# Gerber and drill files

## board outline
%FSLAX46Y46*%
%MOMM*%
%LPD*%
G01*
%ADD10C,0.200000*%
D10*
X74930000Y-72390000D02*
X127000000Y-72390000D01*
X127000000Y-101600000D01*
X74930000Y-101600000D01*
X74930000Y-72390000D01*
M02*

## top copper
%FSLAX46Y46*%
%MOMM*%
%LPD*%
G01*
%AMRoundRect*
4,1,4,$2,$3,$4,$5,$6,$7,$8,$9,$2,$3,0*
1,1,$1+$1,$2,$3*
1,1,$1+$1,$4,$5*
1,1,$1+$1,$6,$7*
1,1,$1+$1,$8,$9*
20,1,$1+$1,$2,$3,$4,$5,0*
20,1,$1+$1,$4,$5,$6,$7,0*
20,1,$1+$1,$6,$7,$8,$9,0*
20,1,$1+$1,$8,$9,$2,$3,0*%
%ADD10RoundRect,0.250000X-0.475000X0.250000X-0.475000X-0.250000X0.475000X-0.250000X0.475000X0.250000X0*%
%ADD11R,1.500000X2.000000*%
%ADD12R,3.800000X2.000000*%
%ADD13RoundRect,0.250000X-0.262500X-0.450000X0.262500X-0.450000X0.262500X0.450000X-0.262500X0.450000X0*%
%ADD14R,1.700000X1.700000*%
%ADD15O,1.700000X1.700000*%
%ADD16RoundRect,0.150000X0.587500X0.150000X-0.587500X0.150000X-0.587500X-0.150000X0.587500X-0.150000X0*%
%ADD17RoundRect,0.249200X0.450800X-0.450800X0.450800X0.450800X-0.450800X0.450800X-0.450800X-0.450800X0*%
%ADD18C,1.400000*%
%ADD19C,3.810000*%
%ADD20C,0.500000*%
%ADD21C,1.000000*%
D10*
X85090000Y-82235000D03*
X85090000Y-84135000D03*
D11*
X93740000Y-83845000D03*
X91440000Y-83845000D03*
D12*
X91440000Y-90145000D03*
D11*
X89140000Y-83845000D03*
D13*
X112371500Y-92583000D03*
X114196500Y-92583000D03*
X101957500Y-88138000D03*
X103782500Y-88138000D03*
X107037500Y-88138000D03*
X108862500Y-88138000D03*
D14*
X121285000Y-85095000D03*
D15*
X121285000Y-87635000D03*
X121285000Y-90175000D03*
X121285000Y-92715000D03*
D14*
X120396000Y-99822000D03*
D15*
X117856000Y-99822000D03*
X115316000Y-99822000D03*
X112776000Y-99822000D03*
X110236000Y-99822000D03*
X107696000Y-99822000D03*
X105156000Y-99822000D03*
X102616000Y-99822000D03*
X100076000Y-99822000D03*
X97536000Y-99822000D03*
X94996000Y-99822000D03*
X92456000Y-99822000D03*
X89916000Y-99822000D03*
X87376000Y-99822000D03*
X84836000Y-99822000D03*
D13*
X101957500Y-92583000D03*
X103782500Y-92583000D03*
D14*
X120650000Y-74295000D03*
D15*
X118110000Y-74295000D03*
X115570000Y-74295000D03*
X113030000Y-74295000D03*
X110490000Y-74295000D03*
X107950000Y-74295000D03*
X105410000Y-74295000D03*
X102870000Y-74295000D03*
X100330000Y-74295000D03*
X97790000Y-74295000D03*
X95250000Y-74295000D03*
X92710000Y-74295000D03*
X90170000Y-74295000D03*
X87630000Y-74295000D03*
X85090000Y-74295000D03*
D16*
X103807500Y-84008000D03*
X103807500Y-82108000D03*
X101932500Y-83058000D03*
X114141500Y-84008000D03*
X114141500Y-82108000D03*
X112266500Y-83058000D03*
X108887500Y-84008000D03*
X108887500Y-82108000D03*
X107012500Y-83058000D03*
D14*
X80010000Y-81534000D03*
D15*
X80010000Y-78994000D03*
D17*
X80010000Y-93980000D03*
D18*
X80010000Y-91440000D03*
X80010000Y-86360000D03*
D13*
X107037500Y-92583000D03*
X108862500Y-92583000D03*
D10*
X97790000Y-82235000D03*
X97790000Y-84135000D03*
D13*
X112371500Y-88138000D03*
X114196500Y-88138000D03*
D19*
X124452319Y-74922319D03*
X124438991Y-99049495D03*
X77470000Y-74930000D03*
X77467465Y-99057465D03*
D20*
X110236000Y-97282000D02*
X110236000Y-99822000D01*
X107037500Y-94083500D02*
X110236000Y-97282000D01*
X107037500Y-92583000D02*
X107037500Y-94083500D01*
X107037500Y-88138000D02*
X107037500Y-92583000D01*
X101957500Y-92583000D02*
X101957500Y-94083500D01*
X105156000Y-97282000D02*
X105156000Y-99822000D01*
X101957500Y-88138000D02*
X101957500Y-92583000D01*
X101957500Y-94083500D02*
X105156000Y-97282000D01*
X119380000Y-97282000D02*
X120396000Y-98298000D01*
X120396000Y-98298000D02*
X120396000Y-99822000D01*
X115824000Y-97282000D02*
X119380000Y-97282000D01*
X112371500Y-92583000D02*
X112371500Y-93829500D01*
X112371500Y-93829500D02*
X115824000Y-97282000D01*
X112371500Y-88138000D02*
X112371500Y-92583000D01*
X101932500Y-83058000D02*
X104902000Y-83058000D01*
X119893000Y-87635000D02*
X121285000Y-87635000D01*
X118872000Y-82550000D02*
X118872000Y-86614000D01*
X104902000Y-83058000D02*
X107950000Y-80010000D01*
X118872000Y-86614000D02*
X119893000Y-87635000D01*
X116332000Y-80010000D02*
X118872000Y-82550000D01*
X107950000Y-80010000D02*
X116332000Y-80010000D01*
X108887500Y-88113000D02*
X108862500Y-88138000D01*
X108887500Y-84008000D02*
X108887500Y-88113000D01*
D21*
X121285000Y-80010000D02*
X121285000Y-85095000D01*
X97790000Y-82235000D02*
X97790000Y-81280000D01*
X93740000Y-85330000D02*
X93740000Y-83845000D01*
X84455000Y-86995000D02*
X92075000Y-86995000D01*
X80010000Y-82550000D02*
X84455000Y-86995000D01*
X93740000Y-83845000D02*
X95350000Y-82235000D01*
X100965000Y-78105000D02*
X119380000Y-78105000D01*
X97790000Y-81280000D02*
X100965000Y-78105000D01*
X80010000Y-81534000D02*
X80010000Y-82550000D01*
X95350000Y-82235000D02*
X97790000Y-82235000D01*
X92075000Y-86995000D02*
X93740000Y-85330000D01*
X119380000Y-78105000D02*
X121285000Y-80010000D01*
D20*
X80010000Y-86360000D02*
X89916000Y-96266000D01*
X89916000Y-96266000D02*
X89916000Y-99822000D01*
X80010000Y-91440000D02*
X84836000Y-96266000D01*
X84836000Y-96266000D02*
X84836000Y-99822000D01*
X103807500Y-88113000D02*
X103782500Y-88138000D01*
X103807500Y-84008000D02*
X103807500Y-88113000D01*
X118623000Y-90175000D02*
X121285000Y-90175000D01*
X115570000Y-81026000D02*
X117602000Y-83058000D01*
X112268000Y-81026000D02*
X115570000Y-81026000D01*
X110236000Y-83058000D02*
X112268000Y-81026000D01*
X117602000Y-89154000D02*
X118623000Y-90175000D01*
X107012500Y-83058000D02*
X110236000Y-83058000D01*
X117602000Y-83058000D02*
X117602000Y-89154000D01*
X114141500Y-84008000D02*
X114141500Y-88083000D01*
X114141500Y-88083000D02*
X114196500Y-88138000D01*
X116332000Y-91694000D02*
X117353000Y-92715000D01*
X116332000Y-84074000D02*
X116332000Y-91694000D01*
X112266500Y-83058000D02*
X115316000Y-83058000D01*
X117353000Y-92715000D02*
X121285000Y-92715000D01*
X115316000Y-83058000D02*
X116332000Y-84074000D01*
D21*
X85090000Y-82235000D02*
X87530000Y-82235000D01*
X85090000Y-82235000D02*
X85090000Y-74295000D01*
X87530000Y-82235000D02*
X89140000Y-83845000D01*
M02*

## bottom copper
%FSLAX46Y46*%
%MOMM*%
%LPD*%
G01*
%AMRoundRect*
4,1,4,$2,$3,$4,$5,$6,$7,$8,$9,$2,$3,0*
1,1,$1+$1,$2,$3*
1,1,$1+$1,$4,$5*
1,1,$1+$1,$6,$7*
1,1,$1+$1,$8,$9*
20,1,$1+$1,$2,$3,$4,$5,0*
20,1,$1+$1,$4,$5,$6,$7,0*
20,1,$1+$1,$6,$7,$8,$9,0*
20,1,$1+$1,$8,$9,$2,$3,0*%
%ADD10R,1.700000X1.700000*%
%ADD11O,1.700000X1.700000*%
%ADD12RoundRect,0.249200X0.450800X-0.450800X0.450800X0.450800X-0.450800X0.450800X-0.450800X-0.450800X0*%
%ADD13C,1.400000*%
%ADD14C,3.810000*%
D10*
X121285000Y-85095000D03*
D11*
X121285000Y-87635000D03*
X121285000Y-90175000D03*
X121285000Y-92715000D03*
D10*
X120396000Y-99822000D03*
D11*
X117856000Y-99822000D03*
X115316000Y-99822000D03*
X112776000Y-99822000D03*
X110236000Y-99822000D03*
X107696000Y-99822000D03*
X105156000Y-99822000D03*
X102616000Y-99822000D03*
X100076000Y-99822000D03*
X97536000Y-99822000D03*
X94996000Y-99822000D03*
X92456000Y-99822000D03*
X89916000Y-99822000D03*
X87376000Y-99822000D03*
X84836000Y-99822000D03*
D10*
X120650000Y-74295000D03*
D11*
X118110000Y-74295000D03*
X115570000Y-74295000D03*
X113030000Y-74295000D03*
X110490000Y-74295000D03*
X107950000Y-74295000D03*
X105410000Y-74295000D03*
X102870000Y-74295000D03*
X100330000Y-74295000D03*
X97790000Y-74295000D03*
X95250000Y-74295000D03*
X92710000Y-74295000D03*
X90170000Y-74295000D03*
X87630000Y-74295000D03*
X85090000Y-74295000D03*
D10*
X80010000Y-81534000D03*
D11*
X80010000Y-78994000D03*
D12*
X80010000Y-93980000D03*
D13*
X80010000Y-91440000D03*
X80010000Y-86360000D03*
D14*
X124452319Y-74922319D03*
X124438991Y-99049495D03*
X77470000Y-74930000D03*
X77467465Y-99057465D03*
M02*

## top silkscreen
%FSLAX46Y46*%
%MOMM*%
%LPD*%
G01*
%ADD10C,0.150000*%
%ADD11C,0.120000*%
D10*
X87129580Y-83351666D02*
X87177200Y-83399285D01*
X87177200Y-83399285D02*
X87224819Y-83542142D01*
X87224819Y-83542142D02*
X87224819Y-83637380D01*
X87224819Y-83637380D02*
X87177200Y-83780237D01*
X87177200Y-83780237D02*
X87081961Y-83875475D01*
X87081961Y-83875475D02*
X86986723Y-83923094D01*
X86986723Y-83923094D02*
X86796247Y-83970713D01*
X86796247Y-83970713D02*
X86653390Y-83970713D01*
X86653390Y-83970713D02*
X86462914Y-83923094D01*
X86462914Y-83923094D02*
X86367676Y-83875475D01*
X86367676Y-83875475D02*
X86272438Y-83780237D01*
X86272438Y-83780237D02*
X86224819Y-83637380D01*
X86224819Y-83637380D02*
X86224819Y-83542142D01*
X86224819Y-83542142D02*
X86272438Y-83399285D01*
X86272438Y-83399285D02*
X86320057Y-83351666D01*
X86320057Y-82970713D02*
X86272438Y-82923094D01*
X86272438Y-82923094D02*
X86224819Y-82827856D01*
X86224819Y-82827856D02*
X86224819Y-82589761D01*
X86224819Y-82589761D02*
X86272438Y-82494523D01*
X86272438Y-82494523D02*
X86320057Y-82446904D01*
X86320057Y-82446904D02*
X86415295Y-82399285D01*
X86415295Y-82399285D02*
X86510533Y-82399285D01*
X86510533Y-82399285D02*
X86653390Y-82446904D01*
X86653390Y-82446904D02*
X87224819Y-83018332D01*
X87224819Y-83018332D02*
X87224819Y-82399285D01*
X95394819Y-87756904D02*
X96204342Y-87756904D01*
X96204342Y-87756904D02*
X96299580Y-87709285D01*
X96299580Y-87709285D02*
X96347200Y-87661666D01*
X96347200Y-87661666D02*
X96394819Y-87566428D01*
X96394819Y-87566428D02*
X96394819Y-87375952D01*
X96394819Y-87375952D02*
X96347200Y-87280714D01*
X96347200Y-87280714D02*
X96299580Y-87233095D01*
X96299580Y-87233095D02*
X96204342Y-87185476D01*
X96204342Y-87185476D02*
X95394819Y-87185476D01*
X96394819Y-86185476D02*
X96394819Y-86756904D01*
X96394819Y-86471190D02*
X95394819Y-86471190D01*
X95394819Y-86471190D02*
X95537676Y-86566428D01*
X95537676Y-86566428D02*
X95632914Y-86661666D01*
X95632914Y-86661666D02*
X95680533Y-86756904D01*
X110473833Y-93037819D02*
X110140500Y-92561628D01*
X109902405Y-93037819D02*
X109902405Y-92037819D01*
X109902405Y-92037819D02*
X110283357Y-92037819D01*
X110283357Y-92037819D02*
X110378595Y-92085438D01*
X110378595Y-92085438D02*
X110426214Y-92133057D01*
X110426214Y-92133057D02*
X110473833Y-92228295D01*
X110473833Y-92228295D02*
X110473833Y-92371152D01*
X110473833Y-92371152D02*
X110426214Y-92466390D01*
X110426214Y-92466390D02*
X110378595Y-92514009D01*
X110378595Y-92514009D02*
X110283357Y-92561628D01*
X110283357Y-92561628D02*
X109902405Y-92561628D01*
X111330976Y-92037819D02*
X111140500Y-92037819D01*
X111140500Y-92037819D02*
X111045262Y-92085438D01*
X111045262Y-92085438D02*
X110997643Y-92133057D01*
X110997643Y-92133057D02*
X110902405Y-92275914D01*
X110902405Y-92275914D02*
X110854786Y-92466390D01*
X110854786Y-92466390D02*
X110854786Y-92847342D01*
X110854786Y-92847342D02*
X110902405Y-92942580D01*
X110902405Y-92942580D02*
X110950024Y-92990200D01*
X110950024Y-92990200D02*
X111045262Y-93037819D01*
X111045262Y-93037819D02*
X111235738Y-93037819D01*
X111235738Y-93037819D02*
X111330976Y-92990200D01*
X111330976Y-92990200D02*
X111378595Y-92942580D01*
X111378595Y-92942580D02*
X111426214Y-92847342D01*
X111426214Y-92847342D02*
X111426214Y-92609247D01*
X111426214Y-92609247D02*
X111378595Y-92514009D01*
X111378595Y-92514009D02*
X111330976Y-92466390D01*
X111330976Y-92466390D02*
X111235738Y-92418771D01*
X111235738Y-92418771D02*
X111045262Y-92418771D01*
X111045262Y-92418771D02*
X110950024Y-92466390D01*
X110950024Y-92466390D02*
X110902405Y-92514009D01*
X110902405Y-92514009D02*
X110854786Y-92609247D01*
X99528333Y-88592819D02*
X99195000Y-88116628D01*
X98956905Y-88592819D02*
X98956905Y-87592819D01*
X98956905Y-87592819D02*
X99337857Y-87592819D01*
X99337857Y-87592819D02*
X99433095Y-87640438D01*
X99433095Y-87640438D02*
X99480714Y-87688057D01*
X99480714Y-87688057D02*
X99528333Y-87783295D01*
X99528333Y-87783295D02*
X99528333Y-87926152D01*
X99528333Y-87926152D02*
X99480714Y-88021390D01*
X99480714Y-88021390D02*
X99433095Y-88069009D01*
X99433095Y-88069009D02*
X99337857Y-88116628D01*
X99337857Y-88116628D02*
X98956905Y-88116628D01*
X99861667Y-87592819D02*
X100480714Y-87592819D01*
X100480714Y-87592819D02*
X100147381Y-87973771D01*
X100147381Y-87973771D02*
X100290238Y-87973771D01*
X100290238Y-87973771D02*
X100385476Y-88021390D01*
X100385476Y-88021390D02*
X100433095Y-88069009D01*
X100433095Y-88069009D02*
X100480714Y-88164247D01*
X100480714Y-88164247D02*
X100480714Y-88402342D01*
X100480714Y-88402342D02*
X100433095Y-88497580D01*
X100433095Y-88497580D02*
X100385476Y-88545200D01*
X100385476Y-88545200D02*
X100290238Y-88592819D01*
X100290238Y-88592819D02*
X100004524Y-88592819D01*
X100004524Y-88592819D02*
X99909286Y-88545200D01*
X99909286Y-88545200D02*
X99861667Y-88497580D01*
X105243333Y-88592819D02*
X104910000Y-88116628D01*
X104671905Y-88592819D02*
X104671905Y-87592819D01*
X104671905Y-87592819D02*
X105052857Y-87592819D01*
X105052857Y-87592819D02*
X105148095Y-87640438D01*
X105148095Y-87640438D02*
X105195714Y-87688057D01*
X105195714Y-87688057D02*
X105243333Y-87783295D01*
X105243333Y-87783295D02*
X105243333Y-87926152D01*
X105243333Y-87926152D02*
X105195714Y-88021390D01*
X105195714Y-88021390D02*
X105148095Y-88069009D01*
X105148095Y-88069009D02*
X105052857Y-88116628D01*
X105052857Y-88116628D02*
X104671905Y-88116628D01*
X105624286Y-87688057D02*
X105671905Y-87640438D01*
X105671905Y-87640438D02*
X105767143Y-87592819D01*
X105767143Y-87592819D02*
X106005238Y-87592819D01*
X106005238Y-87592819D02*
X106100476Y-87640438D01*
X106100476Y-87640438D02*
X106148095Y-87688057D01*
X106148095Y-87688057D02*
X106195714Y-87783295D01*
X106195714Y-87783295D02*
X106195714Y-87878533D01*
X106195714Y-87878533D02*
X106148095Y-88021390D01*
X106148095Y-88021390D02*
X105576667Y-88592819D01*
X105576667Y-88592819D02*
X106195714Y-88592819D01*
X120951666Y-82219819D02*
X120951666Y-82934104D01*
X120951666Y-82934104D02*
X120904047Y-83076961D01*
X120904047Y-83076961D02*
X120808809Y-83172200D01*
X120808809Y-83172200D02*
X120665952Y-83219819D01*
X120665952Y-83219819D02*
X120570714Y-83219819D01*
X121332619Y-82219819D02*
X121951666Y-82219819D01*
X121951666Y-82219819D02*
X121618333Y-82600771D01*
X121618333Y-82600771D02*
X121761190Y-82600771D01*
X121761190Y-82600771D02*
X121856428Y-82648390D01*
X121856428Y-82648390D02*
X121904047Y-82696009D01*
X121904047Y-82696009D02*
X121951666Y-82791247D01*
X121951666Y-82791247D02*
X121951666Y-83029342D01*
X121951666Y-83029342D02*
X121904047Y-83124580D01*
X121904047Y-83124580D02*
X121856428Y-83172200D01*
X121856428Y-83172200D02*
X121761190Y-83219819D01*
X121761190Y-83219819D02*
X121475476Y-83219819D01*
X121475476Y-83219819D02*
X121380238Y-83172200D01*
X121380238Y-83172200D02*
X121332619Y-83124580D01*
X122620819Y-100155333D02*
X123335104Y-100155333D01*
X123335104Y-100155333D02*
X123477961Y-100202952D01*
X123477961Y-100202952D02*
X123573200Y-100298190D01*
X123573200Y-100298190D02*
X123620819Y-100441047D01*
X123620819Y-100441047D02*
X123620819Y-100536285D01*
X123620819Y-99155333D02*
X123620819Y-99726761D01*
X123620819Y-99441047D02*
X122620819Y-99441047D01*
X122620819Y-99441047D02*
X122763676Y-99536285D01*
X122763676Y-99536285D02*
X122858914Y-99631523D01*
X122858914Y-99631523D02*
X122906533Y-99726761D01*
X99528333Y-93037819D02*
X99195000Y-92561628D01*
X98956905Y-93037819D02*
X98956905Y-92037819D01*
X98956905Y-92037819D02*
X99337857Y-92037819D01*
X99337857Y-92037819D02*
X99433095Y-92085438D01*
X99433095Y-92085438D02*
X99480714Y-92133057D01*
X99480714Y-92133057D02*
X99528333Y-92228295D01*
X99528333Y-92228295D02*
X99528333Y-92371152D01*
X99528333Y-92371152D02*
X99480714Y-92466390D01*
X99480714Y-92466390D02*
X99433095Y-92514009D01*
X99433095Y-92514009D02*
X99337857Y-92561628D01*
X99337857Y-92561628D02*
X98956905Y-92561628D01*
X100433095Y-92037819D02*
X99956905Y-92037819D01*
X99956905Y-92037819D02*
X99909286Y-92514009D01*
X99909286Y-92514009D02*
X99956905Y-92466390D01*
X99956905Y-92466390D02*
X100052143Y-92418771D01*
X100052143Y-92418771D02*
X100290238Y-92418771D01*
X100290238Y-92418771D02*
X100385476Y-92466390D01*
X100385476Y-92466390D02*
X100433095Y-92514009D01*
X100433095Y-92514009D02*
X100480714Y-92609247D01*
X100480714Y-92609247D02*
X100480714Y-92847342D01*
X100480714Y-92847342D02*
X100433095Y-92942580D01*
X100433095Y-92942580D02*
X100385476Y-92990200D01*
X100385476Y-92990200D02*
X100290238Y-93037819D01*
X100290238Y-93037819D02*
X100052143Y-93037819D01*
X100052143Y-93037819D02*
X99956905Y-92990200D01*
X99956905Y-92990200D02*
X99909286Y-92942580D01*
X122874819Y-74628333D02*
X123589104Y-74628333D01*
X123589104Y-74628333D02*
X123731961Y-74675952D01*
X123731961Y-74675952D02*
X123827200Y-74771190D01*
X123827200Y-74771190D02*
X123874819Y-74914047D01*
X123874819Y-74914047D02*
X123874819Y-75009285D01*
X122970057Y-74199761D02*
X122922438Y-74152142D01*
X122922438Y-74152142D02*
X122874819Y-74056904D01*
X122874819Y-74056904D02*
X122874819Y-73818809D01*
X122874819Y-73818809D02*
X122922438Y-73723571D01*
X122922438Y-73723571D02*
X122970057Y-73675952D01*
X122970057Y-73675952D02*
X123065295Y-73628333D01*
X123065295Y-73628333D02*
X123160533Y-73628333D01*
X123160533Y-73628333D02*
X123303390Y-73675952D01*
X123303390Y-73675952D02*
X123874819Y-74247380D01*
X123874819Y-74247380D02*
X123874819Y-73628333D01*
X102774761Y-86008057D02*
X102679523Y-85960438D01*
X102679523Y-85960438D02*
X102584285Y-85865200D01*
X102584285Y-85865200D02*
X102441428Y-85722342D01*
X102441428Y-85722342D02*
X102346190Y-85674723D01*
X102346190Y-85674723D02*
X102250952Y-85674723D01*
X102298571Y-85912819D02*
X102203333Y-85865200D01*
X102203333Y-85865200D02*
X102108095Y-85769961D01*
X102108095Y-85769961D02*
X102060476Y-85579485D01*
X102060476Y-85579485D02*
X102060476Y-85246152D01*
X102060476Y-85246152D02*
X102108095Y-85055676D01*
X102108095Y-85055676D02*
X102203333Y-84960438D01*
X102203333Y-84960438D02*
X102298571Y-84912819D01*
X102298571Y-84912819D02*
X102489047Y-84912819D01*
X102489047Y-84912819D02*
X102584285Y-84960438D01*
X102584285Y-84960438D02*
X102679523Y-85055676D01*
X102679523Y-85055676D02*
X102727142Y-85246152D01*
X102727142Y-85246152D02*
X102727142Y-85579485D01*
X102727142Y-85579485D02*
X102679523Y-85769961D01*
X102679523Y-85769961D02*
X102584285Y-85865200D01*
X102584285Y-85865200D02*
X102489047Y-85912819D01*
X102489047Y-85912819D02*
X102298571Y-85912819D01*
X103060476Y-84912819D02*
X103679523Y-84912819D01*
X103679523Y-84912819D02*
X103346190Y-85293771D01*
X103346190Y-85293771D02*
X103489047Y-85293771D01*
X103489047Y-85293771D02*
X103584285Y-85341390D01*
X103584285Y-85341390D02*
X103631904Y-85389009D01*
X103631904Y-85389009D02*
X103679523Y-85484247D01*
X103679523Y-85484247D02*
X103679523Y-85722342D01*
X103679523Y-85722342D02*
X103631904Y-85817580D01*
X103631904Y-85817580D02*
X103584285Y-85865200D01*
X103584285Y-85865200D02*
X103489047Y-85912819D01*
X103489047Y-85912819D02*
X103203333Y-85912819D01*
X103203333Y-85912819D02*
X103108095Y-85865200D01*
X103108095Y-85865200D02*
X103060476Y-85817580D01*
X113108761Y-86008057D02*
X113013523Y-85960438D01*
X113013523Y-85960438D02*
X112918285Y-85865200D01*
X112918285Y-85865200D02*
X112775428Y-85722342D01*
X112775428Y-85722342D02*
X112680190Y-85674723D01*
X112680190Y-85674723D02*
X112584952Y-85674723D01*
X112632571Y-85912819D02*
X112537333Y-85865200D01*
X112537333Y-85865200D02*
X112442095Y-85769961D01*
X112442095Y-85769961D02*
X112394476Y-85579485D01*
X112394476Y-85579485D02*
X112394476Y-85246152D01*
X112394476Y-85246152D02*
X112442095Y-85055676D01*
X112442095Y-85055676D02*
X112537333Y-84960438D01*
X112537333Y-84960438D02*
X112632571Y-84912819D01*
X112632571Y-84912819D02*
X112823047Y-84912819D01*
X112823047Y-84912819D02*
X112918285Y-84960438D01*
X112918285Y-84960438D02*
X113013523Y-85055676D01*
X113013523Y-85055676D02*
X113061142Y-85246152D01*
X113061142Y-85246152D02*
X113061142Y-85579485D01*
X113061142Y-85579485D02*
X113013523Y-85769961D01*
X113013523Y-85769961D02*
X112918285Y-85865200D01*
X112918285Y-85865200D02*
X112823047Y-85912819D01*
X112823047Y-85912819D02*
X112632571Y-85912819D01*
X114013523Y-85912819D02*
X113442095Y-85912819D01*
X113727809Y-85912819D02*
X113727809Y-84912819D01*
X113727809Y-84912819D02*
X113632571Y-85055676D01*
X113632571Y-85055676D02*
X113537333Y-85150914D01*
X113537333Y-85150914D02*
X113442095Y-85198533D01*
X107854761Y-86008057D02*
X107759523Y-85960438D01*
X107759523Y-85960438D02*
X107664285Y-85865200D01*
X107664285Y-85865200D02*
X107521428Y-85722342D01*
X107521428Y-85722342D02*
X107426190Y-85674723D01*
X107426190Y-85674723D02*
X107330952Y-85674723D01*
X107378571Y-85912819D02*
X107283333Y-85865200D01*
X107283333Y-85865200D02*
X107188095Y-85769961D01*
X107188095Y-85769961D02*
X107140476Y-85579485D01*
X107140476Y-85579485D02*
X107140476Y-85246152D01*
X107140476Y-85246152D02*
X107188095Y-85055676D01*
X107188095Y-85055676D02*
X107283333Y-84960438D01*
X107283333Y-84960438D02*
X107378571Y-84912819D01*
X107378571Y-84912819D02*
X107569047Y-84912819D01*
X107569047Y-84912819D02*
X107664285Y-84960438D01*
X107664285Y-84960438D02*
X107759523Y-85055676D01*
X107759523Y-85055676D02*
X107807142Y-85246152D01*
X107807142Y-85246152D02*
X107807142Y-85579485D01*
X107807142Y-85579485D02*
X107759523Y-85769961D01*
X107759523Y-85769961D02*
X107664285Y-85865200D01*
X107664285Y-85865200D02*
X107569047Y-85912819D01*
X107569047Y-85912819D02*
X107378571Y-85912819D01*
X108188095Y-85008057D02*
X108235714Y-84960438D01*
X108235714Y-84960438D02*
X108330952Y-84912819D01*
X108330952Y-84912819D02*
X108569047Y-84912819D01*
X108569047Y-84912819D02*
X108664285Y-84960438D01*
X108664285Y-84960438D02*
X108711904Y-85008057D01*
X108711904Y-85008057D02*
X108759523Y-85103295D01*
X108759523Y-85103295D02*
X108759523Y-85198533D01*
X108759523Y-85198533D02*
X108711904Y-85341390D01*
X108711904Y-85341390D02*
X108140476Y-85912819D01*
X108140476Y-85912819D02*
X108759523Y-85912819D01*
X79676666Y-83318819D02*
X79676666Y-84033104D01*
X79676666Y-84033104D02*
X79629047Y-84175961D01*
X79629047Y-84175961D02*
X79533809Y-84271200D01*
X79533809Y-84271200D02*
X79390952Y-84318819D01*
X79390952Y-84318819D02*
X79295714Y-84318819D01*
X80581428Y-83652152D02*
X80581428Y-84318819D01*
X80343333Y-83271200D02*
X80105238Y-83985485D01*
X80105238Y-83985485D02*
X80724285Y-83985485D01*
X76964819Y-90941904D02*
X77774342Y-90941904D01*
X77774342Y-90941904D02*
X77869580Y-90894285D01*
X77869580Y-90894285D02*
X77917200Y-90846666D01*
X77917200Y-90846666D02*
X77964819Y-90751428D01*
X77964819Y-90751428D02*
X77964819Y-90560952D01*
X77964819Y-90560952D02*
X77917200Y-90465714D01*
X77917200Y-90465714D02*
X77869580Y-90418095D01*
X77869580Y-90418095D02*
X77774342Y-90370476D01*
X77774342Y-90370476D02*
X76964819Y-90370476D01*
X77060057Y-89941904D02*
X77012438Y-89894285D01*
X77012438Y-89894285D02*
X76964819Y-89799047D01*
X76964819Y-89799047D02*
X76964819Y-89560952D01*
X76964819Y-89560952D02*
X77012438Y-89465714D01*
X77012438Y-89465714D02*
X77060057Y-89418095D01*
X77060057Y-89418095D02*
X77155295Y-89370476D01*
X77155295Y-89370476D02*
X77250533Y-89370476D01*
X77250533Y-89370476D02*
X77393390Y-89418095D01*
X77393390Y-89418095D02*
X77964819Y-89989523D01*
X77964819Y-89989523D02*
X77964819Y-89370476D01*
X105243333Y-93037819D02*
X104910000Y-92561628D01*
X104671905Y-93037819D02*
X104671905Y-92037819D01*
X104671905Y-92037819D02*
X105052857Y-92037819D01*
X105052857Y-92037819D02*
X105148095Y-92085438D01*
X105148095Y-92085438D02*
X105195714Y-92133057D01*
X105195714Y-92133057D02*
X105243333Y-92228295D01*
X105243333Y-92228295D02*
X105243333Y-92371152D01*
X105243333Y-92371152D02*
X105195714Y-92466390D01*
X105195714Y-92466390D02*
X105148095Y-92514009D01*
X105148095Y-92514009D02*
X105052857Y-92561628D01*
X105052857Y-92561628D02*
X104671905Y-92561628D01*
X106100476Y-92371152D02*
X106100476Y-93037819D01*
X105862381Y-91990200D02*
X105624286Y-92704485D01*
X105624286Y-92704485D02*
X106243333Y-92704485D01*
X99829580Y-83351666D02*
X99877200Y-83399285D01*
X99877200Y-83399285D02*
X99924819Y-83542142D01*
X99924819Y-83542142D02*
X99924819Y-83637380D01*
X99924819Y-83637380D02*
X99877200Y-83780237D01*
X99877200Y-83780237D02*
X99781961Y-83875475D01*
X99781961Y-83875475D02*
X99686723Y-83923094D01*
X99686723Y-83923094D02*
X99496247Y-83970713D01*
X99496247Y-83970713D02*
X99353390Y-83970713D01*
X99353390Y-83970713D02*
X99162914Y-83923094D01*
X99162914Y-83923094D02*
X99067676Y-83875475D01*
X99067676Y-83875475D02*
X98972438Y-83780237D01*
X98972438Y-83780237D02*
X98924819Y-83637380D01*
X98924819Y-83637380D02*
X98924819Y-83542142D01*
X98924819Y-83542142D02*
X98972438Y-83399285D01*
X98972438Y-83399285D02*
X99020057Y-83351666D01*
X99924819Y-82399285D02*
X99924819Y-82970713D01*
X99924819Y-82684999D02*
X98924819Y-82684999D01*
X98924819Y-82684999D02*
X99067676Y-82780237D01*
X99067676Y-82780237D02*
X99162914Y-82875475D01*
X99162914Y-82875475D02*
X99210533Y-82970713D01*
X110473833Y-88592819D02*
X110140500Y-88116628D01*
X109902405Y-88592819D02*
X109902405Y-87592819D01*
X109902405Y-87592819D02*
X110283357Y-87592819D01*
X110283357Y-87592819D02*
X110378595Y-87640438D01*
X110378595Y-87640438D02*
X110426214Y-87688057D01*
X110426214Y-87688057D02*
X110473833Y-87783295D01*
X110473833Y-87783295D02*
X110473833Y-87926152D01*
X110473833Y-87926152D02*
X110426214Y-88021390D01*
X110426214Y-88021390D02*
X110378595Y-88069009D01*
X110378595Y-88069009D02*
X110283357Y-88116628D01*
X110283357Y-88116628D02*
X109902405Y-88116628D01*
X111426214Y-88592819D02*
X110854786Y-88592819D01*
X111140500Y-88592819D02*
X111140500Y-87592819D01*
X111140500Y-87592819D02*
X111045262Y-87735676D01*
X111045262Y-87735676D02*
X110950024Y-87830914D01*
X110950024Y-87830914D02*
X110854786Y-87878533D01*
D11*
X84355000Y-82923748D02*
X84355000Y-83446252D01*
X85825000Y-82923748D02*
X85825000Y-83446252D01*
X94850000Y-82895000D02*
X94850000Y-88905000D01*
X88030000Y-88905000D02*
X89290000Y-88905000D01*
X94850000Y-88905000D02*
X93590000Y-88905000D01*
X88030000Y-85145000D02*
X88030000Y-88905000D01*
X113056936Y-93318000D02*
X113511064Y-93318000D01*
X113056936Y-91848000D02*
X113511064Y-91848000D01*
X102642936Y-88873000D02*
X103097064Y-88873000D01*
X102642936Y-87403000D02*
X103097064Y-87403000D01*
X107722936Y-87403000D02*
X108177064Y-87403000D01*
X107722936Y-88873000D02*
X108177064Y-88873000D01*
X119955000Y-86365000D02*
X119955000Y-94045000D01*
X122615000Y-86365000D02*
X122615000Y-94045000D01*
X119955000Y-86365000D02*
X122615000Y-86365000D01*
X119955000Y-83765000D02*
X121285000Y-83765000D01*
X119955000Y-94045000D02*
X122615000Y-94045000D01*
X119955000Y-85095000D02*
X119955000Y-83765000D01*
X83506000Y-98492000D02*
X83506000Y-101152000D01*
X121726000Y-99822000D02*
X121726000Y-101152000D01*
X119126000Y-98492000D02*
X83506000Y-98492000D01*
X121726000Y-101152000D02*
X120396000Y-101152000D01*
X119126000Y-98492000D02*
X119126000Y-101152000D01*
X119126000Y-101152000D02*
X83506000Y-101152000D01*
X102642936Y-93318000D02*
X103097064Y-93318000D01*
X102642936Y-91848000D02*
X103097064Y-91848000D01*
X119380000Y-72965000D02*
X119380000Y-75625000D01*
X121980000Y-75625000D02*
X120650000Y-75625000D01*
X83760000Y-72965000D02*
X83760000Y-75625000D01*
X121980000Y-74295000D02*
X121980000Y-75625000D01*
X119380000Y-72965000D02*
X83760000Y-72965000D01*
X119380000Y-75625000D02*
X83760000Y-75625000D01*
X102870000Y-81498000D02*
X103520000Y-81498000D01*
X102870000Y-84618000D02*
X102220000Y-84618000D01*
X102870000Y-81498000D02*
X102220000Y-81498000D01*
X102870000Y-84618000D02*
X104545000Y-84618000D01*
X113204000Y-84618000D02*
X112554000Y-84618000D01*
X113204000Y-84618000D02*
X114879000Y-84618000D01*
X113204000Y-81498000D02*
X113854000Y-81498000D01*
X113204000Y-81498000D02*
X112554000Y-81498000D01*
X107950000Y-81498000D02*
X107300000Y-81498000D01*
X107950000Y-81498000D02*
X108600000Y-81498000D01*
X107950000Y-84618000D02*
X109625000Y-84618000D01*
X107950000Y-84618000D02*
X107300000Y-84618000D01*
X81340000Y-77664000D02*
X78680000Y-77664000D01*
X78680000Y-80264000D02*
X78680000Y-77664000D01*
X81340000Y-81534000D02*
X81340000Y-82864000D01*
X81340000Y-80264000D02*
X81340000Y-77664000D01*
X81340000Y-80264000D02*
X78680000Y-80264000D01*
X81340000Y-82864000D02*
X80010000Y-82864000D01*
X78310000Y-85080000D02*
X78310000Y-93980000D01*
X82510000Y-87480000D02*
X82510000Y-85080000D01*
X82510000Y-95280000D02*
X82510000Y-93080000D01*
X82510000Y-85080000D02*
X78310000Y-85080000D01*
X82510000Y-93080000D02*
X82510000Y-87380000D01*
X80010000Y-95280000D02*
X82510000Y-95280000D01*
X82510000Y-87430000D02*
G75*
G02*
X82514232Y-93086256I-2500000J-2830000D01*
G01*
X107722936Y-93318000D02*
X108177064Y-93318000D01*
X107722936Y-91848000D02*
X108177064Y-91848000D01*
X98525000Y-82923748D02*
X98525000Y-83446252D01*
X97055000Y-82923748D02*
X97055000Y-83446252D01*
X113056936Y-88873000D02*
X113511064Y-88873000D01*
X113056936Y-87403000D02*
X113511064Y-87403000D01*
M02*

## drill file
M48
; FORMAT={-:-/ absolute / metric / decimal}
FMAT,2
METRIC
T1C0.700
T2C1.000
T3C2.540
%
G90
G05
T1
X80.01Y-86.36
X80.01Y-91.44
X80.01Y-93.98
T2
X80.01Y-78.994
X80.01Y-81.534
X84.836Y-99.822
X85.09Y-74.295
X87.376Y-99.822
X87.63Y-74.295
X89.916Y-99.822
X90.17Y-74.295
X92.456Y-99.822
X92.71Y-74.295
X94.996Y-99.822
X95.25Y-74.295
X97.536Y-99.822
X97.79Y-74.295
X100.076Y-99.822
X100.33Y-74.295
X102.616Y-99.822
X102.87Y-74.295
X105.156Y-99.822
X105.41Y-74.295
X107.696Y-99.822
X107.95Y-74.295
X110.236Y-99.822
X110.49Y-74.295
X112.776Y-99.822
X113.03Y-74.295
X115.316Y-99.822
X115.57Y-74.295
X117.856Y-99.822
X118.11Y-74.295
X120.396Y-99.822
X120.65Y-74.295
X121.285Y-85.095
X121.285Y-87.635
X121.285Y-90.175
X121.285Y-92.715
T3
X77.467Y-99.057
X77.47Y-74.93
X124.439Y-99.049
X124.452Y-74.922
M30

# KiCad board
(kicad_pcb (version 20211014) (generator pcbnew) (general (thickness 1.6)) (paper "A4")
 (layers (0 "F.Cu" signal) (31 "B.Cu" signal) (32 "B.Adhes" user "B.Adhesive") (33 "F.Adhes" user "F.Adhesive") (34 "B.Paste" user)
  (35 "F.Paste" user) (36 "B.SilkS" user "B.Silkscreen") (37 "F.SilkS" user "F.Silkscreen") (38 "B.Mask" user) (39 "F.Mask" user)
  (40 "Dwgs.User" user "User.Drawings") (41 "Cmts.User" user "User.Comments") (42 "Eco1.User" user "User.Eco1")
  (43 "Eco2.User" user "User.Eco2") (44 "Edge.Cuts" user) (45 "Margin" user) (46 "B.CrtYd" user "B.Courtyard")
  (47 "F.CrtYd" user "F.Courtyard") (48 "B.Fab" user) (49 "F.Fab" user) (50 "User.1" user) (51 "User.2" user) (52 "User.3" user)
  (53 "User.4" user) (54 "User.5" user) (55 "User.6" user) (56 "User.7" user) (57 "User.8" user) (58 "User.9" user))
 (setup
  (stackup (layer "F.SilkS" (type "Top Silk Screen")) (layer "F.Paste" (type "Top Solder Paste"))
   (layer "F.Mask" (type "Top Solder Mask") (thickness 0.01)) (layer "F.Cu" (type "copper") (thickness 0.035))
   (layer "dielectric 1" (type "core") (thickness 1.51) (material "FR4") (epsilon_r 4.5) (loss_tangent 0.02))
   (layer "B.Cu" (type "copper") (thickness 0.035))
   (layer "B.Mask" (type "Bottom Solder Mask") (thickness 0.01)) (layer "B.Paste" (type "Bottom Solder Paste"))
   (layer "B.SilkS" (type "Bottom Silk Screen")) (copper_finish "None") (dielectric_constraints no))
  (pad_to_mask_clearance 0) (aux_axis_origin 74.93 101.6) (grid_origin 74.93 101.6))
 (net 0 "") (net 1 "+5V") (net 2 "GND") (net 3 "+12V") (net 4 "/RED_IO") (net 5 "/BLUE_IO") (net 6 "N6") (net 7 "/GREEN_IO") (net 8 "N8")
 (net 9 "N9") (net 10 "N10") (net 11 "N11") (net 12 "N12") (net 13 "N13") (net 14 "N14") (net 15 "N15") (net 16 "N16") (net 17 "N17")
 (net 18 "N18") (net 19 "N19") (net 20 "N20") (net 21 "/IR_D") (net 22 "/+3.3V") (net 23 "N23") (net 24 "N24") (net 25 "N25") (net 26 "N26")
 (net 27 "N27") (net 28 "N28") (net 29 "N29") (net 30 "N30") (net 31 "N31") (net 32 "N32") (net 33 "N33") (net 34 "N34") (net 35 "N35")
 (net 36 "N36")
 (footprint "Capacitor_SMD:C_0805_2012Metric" (layer "F.Cu") (at 85.09 83.185 -90)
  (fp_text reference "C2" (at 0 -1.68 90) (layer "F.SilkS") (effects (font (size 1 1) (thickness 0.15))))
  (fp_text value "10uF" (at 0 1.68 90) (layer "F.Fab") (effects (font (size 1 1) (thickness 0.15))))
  (fp_line (start -0.261252 0.735) (end 0.261252 0.735) (layer "F.SilkS") (width 0.12))
  (fp_line (start -0.261252 -0.735) (end 0.261252 -0.735) (layer "F.SilkS") (width 0.12))
  (pad "1" smd roundrect (at -0.95 0 270) (size 1 1.45) (layers "F.Cu" "F.Paste" "F.Mask") (roundrect_rratio 0.25) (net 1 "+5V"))
  (pad "2" smd roundrect (at 0.95 0 270) (size 1 1.45) (layers "F.Cu" "F.Paste" "F.Mask") (roundrect_rratio 0.25) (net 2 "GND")))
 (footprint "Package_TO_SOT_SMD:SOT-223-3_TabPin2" (layer "F.Cu") (at 91.44 86.995 -90)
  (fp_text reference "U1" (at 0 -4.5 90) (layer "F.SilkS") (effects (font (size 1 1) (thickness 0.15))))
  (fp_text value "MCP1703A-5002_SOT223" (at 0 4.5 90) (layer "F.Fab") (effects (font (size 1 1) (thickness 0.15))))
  (fp_line (start -4.1 -3.41) (end 1.91 -3.41) (layer "F.SilkS") (width 0.12))
  (fp_line (start 1.91 3.41) (end 1.91 2.15) (layer "F.SilkS") (width 0.12))
  (fp_line (start 1.91 -3.41) (end 1.91 -2.15) (layer "F.SilkS") (width 0.12))
  (fp_line (start -1.85 3.41) (end 1.91 3.41) (layer "F.SilkS") (width 0.12))
  (pad "1" smd rect (at -3.15 -2.3 270) (size 2 1.5) (layers "F.Cu" "F.Paste" "F.Mask") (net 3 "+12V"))
  (pad "2" smd rect (at -3.15 0 270) (size 2 1.5) (layers "F.Cu" "F.Paste" "F.Mask") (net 2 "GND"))
  (pad "2" smd rect (at 3.15 0 270) (size 2 3.8) (layers "F.Cu" "F.Paste" "F.Mask") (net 2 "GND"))
  (pad "3" smd rect (at -3.15 2.3 270) (size 2 1.5) (layers "F.Cu" "F.Paste" "F.Mask") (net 1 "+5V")))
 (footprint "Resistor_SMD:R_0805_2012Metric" (layer "F.Cu") (at 113.284 92.583)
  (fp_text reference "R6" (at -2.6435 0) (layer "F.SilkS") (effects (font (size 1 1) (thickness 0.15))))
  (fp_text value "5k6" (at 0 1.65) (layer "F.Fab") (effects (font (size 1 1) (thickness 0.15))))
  (fp_line (start -0.227064 0.735) (end 0.227064 0.735) (layer "F.SilkS") (width 0.12))
  (fp_line (start -0.227064 -0.735) (end 0.227064 -0.735) (layer "F.SilkS") (width 0.12))
  (pad "1" smd roundrect (at -0.9125 0) (size 1.025 1.4) (layers "F.Cu" "F.Paste" "F.Mask") (roundrect_rratio 0.243902) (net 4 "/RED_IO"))
  (pad "2" smd roundrect (at 0.9125 0) (size 1.025 1.4) (layers "F.Cu" "F.Paste" "F.Mask") (roundrect_rratio 0.243902) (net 2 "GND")))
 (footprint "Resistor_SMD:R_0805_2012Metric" (layer "F.Cu") (at 102.87 88.138)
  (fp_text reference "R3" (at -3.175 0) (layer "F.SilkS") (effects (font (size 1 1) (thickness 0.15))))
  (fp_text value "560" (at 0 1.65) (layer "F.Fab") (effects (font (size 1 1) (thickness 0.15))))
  (fp_line (start -0.227064 0.735) (end 0.227064 0.735) (layer "F.SilkS") (width 0.12))
  (fp_line (start -0.227064 -0.735) (end 0.227064 -0.735) (layer "F.SilkS") (width 0.12))
  (pad "1" smd roundrect (at -0.9125 0) (size 1.025 1.4) (layers "F.Cu" "F.Paste" "F.Mask") (roundrect_rratio 0.243902) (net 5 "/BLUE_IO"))
  (pad "2" smd roundrect (at 0.9125 0) (size 1.025 1.4) (layers "F.Cu" "F.Paste" "F.Mask") (roundrect_rratio 0.243902) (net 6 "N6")))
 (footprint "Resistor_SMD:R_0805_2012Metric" (layer "F.Cu") (at 107.95 88.138)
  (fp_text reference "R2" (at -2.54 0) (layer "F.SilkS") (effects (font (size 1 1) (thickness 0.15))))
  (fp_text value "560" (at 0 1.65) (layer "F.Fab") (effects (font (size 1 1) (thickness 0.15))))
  (fp_line (start -0.227064 -0.735) (end 0.227064 -0.735) (layer "F.SilkS") (width 0.12))
  (fp_line (start -0.227064 0.735) (end 0.227064 0.735) (layer "F.SilkS") (width 0.12))
  (pad "1" smd roundrect (at -0.9125 0) (size 1.025 1.4) (layers "F.Cu" "F.Paste" "F.Mask") (roundrect_rratio 0.243902) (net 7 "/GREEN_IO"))
  (pad "2" smd roundrect (at 0.9125 0) (size 1.025 1.4) (layers "F.Cu" "F.Paste" "F.Mask") (roundrect_rratio 0.243902) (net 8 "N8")))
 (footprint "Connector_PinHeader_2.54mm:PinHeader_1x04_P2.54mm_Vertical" (layer "F.Cu") (at 121.285 85.095)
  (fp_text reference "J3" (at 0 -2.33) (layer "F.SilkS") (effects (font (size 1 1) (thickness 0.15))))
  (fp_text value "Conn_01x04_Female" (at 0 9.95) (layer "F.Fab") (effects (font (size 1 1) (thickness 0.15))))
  (fp_line (start -1.33 1.27) (end -1.33 8.95) (layer "F.SilkS") (width 0.12))
  (fp_line (start 1.33 1.27) (end 1.33 8.95) (layer "F.SilkS") (width 0.12))
  (fp_line (start -1.33 1.27) (end 1.33 1.27) (layer "F.SilkS") (width 0.12))
  (fp_line (start -1.33 -1.33) (end 0 -1.33) (layer "F.SilkS") (width 0.12))
  (fp_line (start -1.33 8.95) (end 1.33 8.95) (layer "F.SilkS") (width 0.12))
  (fp_line (start -1.33 0) (end -1.33 -1.33) (layer "F.SilkS") (width 0.12))
  (pad "1" thru_hole rect (at 0 0) (size 1.7 1.7) (drill 1) (layers *.Cu *.Mask) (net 3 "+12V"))
  (pad "2" thru_hole oval (at 0 2.54) (size 1.7 1.7) (drill 1) (layers *.Cu *.Mask) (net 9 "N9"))
  (pad "3" thru_hole oval (at 0 5.08) (size 1.7 1.7) (drill 1) (layers *.Cu *.Mask) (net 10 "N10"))
  (pad "4" thru_hole oval (at 0 7.62) (size 1.7 1.7) (drill 1) (layers *.Cu *.Mask) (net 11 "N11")))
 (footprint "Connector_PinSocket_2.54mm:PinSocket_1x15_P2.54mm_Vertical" (layer "F.Cu") (at 120.396 99.822 -90)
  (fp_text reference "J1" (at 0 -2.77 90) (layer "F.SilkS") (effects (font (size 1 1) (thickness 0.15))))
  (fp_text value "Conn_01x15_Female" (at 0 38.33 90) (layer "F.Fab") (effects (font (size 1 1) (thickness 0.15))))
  (fp_line (start -1.33 36.89) (end 1.33 36.89) (layer "F.SilkS") (width 0.12))
  (fp_line (start 0 -1.33) (end 1.33 -1.33) (layer "F.SilkS") (width 0.12))
  (fp_line (start -1.33 1.27) (end -1.33 36.89) (layer "F.SilkS") (width 0.12))
  (fp_line (start 1.33 -1.33) (end 1.33 0) (layer "F.SilkS") (width 0.12))
  (fp_line (start -1.33 1.27) (end 1.33 1.27) (layer "F.SilkS") (width 0.12))
  (fp_line (start 1.33 1.27) (end 1.33 36.89) (layer "F.SilkS") (width 0.12))
  (pad "1" thru_hole rect (at 0 0 270) (size 1.7 1.7) (drill 1) (layers *.Cu *.Mask) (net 4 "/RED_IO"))
  (pad "2" thru_hole oval (at 0 2.54 270) (size 1.7 1.7) (drill 1) (layers *.Cu *.Mask) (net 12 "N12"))
  (pad "3" thru_hole oval (at 0 5.08 270) (size 1.7 1.7) (drill 1) (layers *.Cu *.Mask) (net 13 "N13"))
  (pad "4" thru_hole oval (at 0 7.62 270) (size 1.7 1.7) (drill 1) (layers *.Cu *.Mask) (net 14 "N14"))
  (pad "5" thru_hole oval (at 0 10.16 270) (size 1.7 1.7) (drill 1) (layers *.Cu *.Mask) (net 7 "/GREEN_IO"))
  (pad "6" thru_hole oval (at 0 12.7 270) (size 1.7 1.7) (drill 1) (layers *.Cu *.Mask) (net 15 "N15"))
  (pad "7" thru_hole oval (at 0 15.24 270) (size 1.7 1.7) (drill 1) (layers *.Cu *.Mask) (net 5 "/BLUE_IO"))
  (pad "8" thru_hole oval (at 0 17.78 270) (size 1.7 1.7) (drill 1) (layers *.Cu *.Mask) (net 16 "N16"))
  (pad "9" thru_hole oval (at 0 20.32 270) (size 1.7 1.7) (drill 1) (layers *.Cu *.Mask) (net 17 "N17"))
  (pad "10" thru_hole oval (at 0 22.86 270) (size 1.7 1.7) (drill 1) (layers *.Cu *.Mask) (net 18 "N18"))
  (pad "11" thru_hole oval (at 0 25.4 270) (size 1.7 1.7) (drill 1) (layers *.Cu *.Mask) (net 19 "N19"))
  (pad "12" thru_hole oval (at 0 27.94 270) (size 1.7 1.7) (drill 1) (layers *.Cu *.Mask) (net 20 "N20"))
  (pad "13" thru_hole oval (at 0 30.48 270) (size 1.7 1.7) (drill 1) (layers *.Cu *.Mask) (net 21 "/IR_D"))
  (pad "14" thru_hole oval (at 0 33.02 270) (size 1.7 1.7) (drill 1) (layers *.Cu *.Mask) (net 2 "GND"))
  (pad "15" thru_hole oval (at 0 35.56 270) (size 1.7 1.7) (drill 1) (layers *.Cu *.Mask) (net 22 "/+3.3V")))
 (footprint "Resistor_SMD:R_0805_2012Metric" (layer "F.Cu") (at 102.87 92.583)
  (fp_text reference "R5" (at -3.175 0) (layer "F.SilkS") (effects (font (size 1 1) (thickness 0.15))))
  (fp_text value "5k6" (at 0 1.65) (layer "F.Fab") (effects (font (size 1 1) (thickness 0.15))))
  (fp_line (start -0.227064 0.735) (end 0.227064 0.735) (layer "F.SilkS") (width 0.12))
  (fp_line (start -0.227064 -0.735) (end 0.227064 -0.735) (layer "F.SilkS") (width 0.12))
  (pad "1" smd roundrect (at -0.9125 0) (size 1.025 1.4) (layers "F.Cu" "F.Paste" "F.Mask") (roundrect_rratio 0.243902) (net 5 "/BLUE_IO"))
  (pad "2" smd roundrect (at 0.9125 0) (size 1.025 1.4) (layers "F.Cu" "F.Paste" "F.Mask") (roundrect_rratio 0.243902) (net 2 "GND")))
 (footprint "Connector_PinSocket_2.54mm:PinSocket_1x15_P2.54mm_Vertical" (layer "F.Cu") (at 120.65 74.295 -90)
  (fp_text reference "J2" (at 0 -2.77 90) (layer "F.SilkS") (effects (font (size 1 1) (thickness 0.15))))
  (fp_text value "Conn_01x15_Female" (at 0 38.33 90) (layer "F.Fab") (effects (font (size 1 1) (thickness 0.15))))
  (fp_line (start -1.33 1.27) (end 1.33 1.27) (layer "F.SilkS") (width 0.12))
  (fp_line (start 1.33 -1.33) (end 1.33 0) (layer "F.SilkS") (width 0.12))
  (fp_line (start -1.33 36.89) (end 1.33 36.89) (layer "F.SilkS") (width 0.12))
  (fp_line (start 0 -1.33) (end 1.33 -1.33) (layer "F.SilkS") (width 0.12))
  (fp_line (start -1.33 1.27) (end -1.33 36.89) (layer "F.SilkS") (width 0.12))
  (fp_line (start 1.33 1.27) (end 1.33 36.89) (layer "F.SilkS") (width 0.12))
  (pad "1" thru_hole rect (at 0 0 270) (size 1.7 1.7) (drill 1) (layers *.Cu *.Mask) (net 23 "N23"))
  (pad "2" thru_hole oval (at 0 2.54 270) (size 1.7 1.7) (drill 1) (layers *.Cu *.Mask) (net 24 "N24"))
  (pad "3" thru_hole oval (at 0 5.08 270) (size 1.7 1.7) (drill 1) (layers *.Cu *.Mask) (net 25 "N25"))
  (pad "4" thru_hole oval (at 0 7.62 270) (size 1.7 1.7) (drill 1) (layers *.Cu *.Mask) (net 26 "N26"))
  (pad "5" thru_hole oval (at 0 10.16 270) (size 1.7 1.7) (drill 1) (layers *.Cu *.Mask) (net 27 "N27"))
  (pad "6" thru_hole oval (at 0 12.7 270) (size 1.7 1.7) (drill 1) (layers *.Cu *.Mask) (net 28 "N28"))
  (pad "7" thru_hole oval (at 0 15.24 270) (size 1.7 1.7) (drill 1) (layers *.Cu *.Mask) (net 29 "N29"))
  (pad "8" thru_hole oval (at 0 17.78 270) (size 1.7 1.7) (drill 1) (layers *.Cu *.Mask) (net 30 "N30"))
  (pad "9" thru_hole oval (at 0 20.32 270) (size 1.7 1.7) (drill 1) (layers *.Cu *.Mask) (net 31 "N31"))
  (pad "10" thru_hole oval (at 0 22.86 270) (size 1.7 1.7) (drill 1) (layers *.Cu *.Mask) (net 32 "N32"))
  (pad "11" thru_hole oval (at 0 25.4 270) (size 1.7 1.7) (drill 1) (layers *.Cu *.Mask) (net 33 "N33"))
  (pad "12" thru_hole oval (at 0 27.94 270) (size 1.7 1.7) (drill 1) (layers *.Cu *.Mask) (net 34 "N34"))
  (pad "13" thru_hole oval (at 0 30.48 270) (size 1.7 1.7) (drill 1) (layers *.Cu *.Mask) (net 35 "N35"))
  (pad "14" thru_hole oval (at 0 33.02 270) (size 1.7 1.7) (drill 1) (layers *.Cu *.Mask) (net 2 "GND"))
  (pad "15" thru_hole oval (at 0 35.56 270) (size 1.7 1.7) (drill 1) (layers *.Cu *.Mask) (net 1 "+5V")))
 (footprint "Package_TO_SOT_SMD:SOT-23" (layer "F.Cu") (at 102.87 83.058 180)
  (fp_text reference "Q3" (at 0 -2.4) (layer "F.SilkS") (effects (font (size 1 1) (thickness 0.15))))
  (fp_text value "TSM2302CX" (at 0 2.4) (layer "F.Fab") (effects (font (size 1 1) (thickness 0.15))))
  (fp_line (start 0 1.56) (end -0.65 1.56) (layer "F.SilkS") (width 0.12))
  (fp_line (start 0 -1.56) (end 0.65 -1.56) (layer "F.SilkS") (width 0.12))
  (fp_line (start 0 1.56) (end 0.65 1.56) (layer "F.SilkS") (width 0.12))
  (fp_line (start 0 -1.56) (end -1.675 -1.56) (layer "F.SilkS") (width 0.12))
  (pad "1" smd roundrect (at -0.9375 -0.95 180) (size 1.475 0.6) (layers "F.Cu" "F.Paste" "F.Mask") (roundrect_rratio 0.25) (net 6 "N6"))
  (pad "2" smd roundrect (at -0.9375 0.95 180) (size 1.475 0.6) (layers "F.Cu" "F.Paste" "F.Mask") (roundrect_rratio 0.25) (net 2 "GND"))
  (pad "3" smd roundrect (at 0.9375 0 180) (size 1.475 0.6) (layers "F.Cu" "F.Paste" "F.Mask") (roundrect_rratio 0.25) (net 9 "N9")))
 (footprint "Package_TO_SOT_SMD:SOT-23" (layer "F.Cu") (at 113.204 83.058 180)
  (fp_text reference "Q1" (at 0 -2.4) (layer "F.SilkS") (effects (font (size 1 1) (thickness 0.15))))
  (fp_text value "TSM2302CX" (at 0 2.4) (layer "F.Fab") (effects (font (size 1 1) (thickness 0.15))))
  (fp_line (start 0 -1.56) (end 0.65 -1.56) (layer "F.SilkS") (width 0.12))
  (fp_line (start 0 -1.56) (end -1.675 -1.56) (layer "F.SilkS") (width 0.12))
  (fp_line (start 0 1.56) (end -0.65 1.56) (layer "F.SilkS") (width 0.12))
  (fp_line (start 0 1.56) (end 0.65 1.56) (layer "F.SilkS") (width 0.12))
  (pad "1" smd roundrect (at -0.9375 -0.95 180) (size 1.475 0.6) (layers "F.Cu" "F.Paste" "F.Mask") (roundrect_rratio 0.25) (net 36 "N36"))
  (pad "2" smd roundrect (at -0.9375 0.95 180) (size 1.475 0.6) (layers "F.Cu" "F.Paste" "F.Mask") (roundrect_rratio 0.25) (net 2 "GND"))
  (pad "3" smd roundrect (at 0.9375 0 180) (size 1.475 0.6) (layers "F.Cu" "F.Paste" "F.Mask") (roundrect_rratio 0.25) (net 11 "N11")))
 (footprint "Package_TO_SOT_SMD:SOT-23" (layer "F.Cu") (at 107.95 83.058 180)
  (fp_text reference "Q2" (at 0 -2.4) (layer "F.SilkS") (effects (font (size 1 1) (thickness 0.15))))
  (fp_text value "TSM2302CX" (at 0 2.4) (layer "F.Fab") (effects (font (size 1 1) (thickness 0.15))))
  (fp_line (start 0 1.56) (end 0.65 1.56) (layer "F.SilkS") (width 0.12))
  (fp_line (start 0 1.56) (end -0.65 1.56) (layer "F.SilkS") (width 0.12))
  (fp_line (start 0 -1.56) (end -1.675 -1.56) (layer "F.SilkS") (width 0.12))
  (fp_line (start 0 -1.56) (end 0.65 -1.56) (layer "F.SilkS") (width 0.12))
  (pad "1" smd roundrect (at -0.9375 -0.95 180) (size 1.475 0.6) (layers "F.Cu" "F.Paste" "F.Mask") (roundrect_rratio 0.25) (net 8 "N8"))
  (pad "2" smd roundrect (at -0.9375 0.95 180) (size 1.475 0.6) (layers "F.Cu" "F.Paste" "F.Mask") (roundrect_rratio 0.25) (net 2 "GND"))
  (pad "3" smd roundrect (at 0.9375 0 180) (size 1.475 0.6) (layers "F.Cu" "F.Paste" "F.Mask") (roundrect_rratio 0.25) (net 10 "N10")))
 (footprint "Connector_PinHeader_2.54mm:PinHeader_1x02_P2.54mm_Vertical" (layer "F.Cu") (at 80.01 81.534 180)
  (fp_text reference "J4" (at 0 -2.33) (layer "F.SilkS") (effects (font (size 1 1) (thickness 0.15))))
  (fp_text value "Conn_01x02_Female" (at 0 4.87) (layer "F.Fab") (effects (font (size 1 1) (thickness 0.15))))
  (fp_line (start -1.33 3.87) (end 1.33 3.87) (layer "F.SilkS") (width 0.12))
  (fp_line (start 1.33 1.27) (end 1.33 3.87) (layer "F.SilkS") (width 0.12))
  (fp_line (start -1.33 0) (end -1.33 -1.33) (layer "F.SilkS") (width 0.12))
  (fp_line (start -1.33 1.27) (end -1.33 3.87) (layer "F.SilkS") (width 0.12))
  (fp_line (start -1.33 1.27) (end 1.33 1.27) (layer "F.SilkS") (width 0.12))
  (fp_line (start -1.33 -1.33) (end 0 -1.33) (layer "F.SilkS") (width 0.12))
  (pad "1" thru_hole rect (at 0 0 180) (size 1.7 1.7) (drill 1) (layers *.Cu *.Mask) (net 3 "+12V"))
  (pad "2" thru_hole oval (at 0 2.54 180) (size 1.7 1.7) (drill 1) (layers *.Cu *.Mask) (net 2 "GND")))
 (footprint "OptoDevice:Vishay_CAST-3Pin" (layer "F.Cu") (at 80.01 93.98 90)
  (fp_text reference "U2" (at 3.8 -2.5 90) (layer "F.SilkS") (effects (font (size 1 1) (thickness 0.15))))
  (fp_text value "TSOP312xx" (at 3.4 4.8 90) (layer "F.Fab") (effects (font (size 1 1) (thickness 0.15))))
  (fp_line (start 8.9 -1.7) (end 0 -1.7) (layer "F.SilkS") (width 0.12))
  (fp_line (start 6.5 2.5) (end 8.9 2.5) (layer "F.SilkS") (width 0.12))
  (fp_line (start -1.3 2.5) (end 0.9 2.5) (layer "F.SilkS") (width 0.12))
  (fp_line (start 8.9 2.5) (end 8.9 -1.7) (layer "F.SilkS") (width 0.12))
  (fp_line (start 0.9 2.5) (end 6.6 2.5) (layer "F.SilkS") (width 0.12))
  (fp_line (start -1.3 0) (end -1.3 2.5) (layer "F.SilkS") (width 0.12))
  (fp_arc (start 6.55 2.5) (mid 3.722825 3.776095) (end 0.893744 2.504232) (layer "F.SilkS") (width 0.12))
  (pad "1" thru_hole roundrect (at 0 0 90) (size 1.4 1.4) (drill 0.7) (layers *.Cu *.Mask) (roundrect_rratio 0.178) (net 2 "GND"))
  (pad "2" thru_hole circle (at 2.54 0 90) (size 1.4 1.4) (drill 0.7) (layers *.Cu *.Mask) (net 22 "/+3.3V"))
  (pad "3" thru_hole circle (at 7.62 0 90) (size 1.4 1.4) (drill 0.7) (layers *.Cu *.Mask) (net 21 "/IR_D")))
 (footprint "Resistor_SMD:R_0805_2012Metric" (layer "F.Cu") (at 107.95 92.583)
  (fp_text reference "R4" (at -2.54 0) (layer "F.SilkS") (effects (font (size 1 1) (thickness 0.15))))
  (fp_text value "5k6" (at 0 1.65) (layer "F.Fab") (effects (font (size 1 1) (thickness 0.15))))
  (fp_line (start -0.227064 0.735) (end 0.227064 0.735) (layer "F.SilkS") (width 0.12))
  (fp_line (start -0.227064 -0.735) (end 0.227064 -0.735) (layer "F.SilkS") (width 0.12))
  (pad "1" smd roundrect (at -0.9125 0) (size 1.025 1.4) (layers "F.Cu" "F.Paste" "F.Mask") (roundrect_rratio 0.243902) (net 7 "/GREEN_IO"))
  (pad "2" smd roundrect (at 0.9125 0) (size 1.025 1.4) (layers "F.Cu" "F.Paste" "F.Mask") (roundrect_rratio 0.243902) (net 2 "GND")))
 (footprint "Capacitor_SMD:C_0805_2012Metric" (layer "F.Cu") (at 97.79 83.185 -90)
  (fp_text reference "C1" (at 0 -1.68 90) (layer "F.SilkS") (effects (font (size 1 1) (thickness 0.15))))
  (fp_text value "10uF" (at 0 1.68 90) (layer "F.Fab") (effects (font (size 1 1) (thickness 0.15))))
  (fp_line (start -0.261252 -0.735) (end 0.261252 -0.735) (layer "F.SilkS") (width 0.12))
  (fp_line (start -0.261252 0.735) (end 0.261252 0.735) (layer "F.SilkS") (width 0.12))
  (pad "1" smd roundrect (at -0.95 0 270) (size 1 1.45) (layers "F.Cu" "F.Paste" "F.Mask") (roundrect_rratio 0.25) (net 3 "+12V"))
  (pad "2" smd roundrect (at 0.95 0 270) (size 1 1.45) (layers "F.Cu" "F.Paste" "F.Mask") (roundrect_rratio 0.25) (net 2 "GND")))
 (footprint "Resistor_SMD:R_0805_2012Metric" (layer "F.Cu") (at 113.284 88.138)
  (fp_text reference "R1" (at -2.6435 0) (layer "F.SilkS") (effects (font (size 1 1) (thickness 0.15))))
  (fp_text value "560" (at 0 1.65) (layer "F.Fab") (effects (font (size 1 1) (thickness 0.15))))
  (fp_line (start -0.227064 0.735) (end 0.227064 0.735) (layer "F.SilkS") (width 0.12))
  (fp_line (start -0.227064 -0.735) (end 0.227064 -0.735) (layer "F.SilkS") (width 0.12))
  (pad "1" smd roundrect (at -0.9125 0) (size 1.025 1.4) (layers "F.Cu" "F.Paste" "F.Mask") (roundrect_rratio 0.243902) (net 4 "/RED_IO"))
  (pad "2" smd roundrect (at 0.9125 0) (size 1.025 1.4) (layers "F.Cu" "F.Paste" "F.Mask") (roundrect_rratio 0.243902) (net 36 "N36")))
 (gr_rect (start 74.93 101.6) (end 127 72.39) (layer "Edge.Cuts") (width 0.2) (fill none))
 (via (at 124.452319 74.922319) (size 3.81) (drill 2.54) (layers "F.Cu" "B.Cu") (free) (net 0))
 (via (at 124.438991 99.049495) (size 3.81) (drill 2.54) (layers "F.Cu" "B.Cu") (free) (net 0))
 (via (at 77.47 74.93) (size 3.81) (drill 2.54) (layers "F.Cu" "B.Cu") (free) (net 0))
 (via (at 77.467465 99.057465) (size 3.81) (drill 2.54) (layers "F.Cu" "B.Cu") (free) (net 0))
 (segment (start 110.236 97.282) (end 110.236 99.822) (width 0.5) (layer "F.Cu") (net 7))
 (segment (start 107.0375 94.0835) (end 110.236 97.282) (width 0.5) (layer "F.Cu") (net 7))
 (segment (start 107.0375 92.583) (end 107.0375 94.0835) (width 0.5) (layer "F.Cu") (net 7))
 (segment (start 107.0375 88.138) (end 107.0375 92.583) (width 0.5) (layer "F.Cu") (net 7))
 (segment (start 101.9575 92.583) (end 101.9575 94.0835) (width 0.5) (layer "F.Cu") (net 5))
 (segment (start 105.156 97.282) (end 105.156 99.822) (width 0.5) (layer "F.Cu") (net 5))
 (segment (start 101.9575 88.138) (end 101.9575 92.583) (width 0.5) (layer "F.Cu") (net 5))
 (segment (start 101.9575 94.0835) (end 105.156 97.282) (width 0.5) (layer "F.Cu") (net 5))
 (segment (start 119.38 97.282) (end 120.396 98.298) (width 0.5) (layer "F.Cu") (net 4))
 (segment (start 120.396 98.298) (end 120.396 99.822) (width 0.5) (layer "F.Cu") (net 4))
 (segment (start 115.824 97.282) (end 119.38 97.282) (width 0.5) (layer "F.Cu") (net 4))
 (segment (start 112.3715 92.583) (end 112.3715 93.8295) (width 0.5) (layer "F.Cu") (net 4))
 (segment (start 112.3715 93.8295) (end 115.824 97.282) (width 0.5) (layer "F.Cu") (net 4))
 (segment (start 112.3715 88.138) (end 112.3715 92.583) (width 0.5) (layer "F.Cu") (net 4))
 (segment (start 101.9325 83.058) (end 104.902 83.058) (width 0.5) (layer "F.Cu") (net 9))
 (segment (start 119.893 87.635) (end 121.285 87.635) (width 0.5) (layer "F.Cu") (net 9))
 (segment (start 118.872 82.55) (end 118.872 86.614) (width 0.5) (layer "F.Cu") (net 9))
 (segment (start 104.902 83.058) (end 107.95 80.01) (width 0.5) (layer "F.Cu") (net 9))
 (segment (start 118.872 86.614) (end 119.893 87.635) (width 0.5) (layer "F.Cu") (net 9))
 (segment (start 116.332 80.01) (end 118.872 82.55) (width 0.5) (layer "F.Cu") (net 9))
 (segment (start 107.95 80.01) (end 116.332 80.01) (width 0.5) (layer "F.Cu") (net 9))
 (segment (start 108.8875 88.113) (end 108.8625 88.138) (width 0.5) (layer "F.Cu") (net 8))
 (segment (start 108.8875 84.008) (end 108.8875 88.113) (width 0.5) (layer "F.Cu") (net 8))
 (segment (start 121.285 80.01) (end 121.285 85.095) (width 1) (layer "F.Cu") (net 3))
 (segment (start 97.79 82.235) (end 97.79 81.28) (width 1) (layer "F.Cu") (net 3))
 (segment (start 93.74 85.33) (end 93.74 83.845) (width 1) (layer "F.Cu") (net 3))
 (segment (start 84.455 86.995) (end 92.075 86.995) (width 1) (layer "F.Cu") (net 3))
 (segment (start 80.01 82.55) (end 84.455 86.995) (width 1) (layer "F.Cu") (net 3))
 (segment (start 93.74 83.845) (end 95.35 82.235) (width 1) (layer "F.Cu") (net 3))
 (segment (start 100.965 78.105) (end 119.38 78.105) (width 1) (layer "F.Cu") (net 3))
 (segment (start 97.79 81.28) (end 100.965 78.105) (width 1) (layer "F.Cu") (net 3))
 (segment (start 80.01 81.534) (end 80.01 82.55) (width 1) (layer "F.Cu") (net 3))
 (segment (start 95.35 82.235) (end 97.79 82.235) (width 1) (layer "F.Cu") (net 3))
 (segment (start 92.075 86.995) (end 93.74 85.33) (width 1) (layer "F.Cu") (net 3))
 (segment (start 119.38 78.105) (end 121.285 80.01) (width 1) (layer "F.Cu") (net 3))
 (segment (start 80.01 86.36) (end 89.916 96.266) (width 0.5) (layer "F.Cu") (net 21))
 (segment (start 89.916 96.266) (end 89.916 99.822) (width 0.5) (layer "F.Cu") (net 21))
 (segment (start 80.01 91.44) (end 84.836 96.266) (width 0.5) (layer "F.Cu") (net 22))
 (segment (start 84.836 96.266) (end 84.836 99.822) (width 0.5) (layer "F.Cu") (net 22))
 (segment (start 103.8075 88.113) (end 103.7825 88.138) (width 0.5) (layer "F.Cu") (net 6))
 (segment (start 103.8075 84.008) (end 103.8075 88.113) (width 0.5) (layer "F.Cu") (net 6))
 (segment (start 118.623 90.175) (end 121.285 90.175) (width 0.5) (layer "F.Cu") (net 10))
 (segment (start 115.57 81.026) (end 117.602 83.058) (width 0.5) (layer "F.Cu") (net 10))
 (segment (start 112.268 81.026) (end 115.57 81.026) (width 0.5) (layer "F.Cu") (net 10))
 (segment (start 110.236 83.058) (end 112.268 81.026) (width 0.5) (layer "F.Cu") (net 10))
 (segment (start 117.602 89.154) (end 118.623 90.175) (width 0.5) (layer "F.Cu") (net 10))
 (segment (start 107.0125 83.058) (end 110.236 83.058) (width 0.5) (layer "F.Cu") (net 10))
 (segment (start 117.602 83.058) (end 117.602 89.154) (width 0.5) (layer "F.Cu") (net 10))
 (segment (start 114.1415 84.008) (end 114.1415 88.083) (width 0.5) (layer "F.Cu") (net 36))
 (segment (start 114.1415 88.083) (end 114.1965 88.138) (width 0.5) (layer "F.Cu") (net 36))
 (segment (start 116.332 91.694) (end 117.353 92.715) (width 0.5) (layer "F.Cu") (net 11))
 (segment (start 116.332 84.074) (end 116.332 91.694) (width 0.5) (layer "F.Cu") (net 11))
 (segment (start 112.2665 83.058) (end 115.316 83.058) (width 0.5) (layer "F.Cu") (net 11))
 (segment (start 117.353 92.715) (end 121.285 92.715) (width 0.5) (layer "F.Cu") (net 11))
 (segment (start 115.316 83.058) (end 116.332 84.074) (width 0.5) (layer "F.Cu") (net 11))
 (segment (start 85.09 82.235) (end 87.53 82.235) (width 1) (layer "F.Cu") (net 1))
 (segment (start 85.09 82.235) (end 85.09 74.295) (width 1) (layer "F.Cu") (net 1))
 (segment (start 87.53 82.235) (end 89.14 83.845) (width 1) (layer "F.Cu") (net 1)))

